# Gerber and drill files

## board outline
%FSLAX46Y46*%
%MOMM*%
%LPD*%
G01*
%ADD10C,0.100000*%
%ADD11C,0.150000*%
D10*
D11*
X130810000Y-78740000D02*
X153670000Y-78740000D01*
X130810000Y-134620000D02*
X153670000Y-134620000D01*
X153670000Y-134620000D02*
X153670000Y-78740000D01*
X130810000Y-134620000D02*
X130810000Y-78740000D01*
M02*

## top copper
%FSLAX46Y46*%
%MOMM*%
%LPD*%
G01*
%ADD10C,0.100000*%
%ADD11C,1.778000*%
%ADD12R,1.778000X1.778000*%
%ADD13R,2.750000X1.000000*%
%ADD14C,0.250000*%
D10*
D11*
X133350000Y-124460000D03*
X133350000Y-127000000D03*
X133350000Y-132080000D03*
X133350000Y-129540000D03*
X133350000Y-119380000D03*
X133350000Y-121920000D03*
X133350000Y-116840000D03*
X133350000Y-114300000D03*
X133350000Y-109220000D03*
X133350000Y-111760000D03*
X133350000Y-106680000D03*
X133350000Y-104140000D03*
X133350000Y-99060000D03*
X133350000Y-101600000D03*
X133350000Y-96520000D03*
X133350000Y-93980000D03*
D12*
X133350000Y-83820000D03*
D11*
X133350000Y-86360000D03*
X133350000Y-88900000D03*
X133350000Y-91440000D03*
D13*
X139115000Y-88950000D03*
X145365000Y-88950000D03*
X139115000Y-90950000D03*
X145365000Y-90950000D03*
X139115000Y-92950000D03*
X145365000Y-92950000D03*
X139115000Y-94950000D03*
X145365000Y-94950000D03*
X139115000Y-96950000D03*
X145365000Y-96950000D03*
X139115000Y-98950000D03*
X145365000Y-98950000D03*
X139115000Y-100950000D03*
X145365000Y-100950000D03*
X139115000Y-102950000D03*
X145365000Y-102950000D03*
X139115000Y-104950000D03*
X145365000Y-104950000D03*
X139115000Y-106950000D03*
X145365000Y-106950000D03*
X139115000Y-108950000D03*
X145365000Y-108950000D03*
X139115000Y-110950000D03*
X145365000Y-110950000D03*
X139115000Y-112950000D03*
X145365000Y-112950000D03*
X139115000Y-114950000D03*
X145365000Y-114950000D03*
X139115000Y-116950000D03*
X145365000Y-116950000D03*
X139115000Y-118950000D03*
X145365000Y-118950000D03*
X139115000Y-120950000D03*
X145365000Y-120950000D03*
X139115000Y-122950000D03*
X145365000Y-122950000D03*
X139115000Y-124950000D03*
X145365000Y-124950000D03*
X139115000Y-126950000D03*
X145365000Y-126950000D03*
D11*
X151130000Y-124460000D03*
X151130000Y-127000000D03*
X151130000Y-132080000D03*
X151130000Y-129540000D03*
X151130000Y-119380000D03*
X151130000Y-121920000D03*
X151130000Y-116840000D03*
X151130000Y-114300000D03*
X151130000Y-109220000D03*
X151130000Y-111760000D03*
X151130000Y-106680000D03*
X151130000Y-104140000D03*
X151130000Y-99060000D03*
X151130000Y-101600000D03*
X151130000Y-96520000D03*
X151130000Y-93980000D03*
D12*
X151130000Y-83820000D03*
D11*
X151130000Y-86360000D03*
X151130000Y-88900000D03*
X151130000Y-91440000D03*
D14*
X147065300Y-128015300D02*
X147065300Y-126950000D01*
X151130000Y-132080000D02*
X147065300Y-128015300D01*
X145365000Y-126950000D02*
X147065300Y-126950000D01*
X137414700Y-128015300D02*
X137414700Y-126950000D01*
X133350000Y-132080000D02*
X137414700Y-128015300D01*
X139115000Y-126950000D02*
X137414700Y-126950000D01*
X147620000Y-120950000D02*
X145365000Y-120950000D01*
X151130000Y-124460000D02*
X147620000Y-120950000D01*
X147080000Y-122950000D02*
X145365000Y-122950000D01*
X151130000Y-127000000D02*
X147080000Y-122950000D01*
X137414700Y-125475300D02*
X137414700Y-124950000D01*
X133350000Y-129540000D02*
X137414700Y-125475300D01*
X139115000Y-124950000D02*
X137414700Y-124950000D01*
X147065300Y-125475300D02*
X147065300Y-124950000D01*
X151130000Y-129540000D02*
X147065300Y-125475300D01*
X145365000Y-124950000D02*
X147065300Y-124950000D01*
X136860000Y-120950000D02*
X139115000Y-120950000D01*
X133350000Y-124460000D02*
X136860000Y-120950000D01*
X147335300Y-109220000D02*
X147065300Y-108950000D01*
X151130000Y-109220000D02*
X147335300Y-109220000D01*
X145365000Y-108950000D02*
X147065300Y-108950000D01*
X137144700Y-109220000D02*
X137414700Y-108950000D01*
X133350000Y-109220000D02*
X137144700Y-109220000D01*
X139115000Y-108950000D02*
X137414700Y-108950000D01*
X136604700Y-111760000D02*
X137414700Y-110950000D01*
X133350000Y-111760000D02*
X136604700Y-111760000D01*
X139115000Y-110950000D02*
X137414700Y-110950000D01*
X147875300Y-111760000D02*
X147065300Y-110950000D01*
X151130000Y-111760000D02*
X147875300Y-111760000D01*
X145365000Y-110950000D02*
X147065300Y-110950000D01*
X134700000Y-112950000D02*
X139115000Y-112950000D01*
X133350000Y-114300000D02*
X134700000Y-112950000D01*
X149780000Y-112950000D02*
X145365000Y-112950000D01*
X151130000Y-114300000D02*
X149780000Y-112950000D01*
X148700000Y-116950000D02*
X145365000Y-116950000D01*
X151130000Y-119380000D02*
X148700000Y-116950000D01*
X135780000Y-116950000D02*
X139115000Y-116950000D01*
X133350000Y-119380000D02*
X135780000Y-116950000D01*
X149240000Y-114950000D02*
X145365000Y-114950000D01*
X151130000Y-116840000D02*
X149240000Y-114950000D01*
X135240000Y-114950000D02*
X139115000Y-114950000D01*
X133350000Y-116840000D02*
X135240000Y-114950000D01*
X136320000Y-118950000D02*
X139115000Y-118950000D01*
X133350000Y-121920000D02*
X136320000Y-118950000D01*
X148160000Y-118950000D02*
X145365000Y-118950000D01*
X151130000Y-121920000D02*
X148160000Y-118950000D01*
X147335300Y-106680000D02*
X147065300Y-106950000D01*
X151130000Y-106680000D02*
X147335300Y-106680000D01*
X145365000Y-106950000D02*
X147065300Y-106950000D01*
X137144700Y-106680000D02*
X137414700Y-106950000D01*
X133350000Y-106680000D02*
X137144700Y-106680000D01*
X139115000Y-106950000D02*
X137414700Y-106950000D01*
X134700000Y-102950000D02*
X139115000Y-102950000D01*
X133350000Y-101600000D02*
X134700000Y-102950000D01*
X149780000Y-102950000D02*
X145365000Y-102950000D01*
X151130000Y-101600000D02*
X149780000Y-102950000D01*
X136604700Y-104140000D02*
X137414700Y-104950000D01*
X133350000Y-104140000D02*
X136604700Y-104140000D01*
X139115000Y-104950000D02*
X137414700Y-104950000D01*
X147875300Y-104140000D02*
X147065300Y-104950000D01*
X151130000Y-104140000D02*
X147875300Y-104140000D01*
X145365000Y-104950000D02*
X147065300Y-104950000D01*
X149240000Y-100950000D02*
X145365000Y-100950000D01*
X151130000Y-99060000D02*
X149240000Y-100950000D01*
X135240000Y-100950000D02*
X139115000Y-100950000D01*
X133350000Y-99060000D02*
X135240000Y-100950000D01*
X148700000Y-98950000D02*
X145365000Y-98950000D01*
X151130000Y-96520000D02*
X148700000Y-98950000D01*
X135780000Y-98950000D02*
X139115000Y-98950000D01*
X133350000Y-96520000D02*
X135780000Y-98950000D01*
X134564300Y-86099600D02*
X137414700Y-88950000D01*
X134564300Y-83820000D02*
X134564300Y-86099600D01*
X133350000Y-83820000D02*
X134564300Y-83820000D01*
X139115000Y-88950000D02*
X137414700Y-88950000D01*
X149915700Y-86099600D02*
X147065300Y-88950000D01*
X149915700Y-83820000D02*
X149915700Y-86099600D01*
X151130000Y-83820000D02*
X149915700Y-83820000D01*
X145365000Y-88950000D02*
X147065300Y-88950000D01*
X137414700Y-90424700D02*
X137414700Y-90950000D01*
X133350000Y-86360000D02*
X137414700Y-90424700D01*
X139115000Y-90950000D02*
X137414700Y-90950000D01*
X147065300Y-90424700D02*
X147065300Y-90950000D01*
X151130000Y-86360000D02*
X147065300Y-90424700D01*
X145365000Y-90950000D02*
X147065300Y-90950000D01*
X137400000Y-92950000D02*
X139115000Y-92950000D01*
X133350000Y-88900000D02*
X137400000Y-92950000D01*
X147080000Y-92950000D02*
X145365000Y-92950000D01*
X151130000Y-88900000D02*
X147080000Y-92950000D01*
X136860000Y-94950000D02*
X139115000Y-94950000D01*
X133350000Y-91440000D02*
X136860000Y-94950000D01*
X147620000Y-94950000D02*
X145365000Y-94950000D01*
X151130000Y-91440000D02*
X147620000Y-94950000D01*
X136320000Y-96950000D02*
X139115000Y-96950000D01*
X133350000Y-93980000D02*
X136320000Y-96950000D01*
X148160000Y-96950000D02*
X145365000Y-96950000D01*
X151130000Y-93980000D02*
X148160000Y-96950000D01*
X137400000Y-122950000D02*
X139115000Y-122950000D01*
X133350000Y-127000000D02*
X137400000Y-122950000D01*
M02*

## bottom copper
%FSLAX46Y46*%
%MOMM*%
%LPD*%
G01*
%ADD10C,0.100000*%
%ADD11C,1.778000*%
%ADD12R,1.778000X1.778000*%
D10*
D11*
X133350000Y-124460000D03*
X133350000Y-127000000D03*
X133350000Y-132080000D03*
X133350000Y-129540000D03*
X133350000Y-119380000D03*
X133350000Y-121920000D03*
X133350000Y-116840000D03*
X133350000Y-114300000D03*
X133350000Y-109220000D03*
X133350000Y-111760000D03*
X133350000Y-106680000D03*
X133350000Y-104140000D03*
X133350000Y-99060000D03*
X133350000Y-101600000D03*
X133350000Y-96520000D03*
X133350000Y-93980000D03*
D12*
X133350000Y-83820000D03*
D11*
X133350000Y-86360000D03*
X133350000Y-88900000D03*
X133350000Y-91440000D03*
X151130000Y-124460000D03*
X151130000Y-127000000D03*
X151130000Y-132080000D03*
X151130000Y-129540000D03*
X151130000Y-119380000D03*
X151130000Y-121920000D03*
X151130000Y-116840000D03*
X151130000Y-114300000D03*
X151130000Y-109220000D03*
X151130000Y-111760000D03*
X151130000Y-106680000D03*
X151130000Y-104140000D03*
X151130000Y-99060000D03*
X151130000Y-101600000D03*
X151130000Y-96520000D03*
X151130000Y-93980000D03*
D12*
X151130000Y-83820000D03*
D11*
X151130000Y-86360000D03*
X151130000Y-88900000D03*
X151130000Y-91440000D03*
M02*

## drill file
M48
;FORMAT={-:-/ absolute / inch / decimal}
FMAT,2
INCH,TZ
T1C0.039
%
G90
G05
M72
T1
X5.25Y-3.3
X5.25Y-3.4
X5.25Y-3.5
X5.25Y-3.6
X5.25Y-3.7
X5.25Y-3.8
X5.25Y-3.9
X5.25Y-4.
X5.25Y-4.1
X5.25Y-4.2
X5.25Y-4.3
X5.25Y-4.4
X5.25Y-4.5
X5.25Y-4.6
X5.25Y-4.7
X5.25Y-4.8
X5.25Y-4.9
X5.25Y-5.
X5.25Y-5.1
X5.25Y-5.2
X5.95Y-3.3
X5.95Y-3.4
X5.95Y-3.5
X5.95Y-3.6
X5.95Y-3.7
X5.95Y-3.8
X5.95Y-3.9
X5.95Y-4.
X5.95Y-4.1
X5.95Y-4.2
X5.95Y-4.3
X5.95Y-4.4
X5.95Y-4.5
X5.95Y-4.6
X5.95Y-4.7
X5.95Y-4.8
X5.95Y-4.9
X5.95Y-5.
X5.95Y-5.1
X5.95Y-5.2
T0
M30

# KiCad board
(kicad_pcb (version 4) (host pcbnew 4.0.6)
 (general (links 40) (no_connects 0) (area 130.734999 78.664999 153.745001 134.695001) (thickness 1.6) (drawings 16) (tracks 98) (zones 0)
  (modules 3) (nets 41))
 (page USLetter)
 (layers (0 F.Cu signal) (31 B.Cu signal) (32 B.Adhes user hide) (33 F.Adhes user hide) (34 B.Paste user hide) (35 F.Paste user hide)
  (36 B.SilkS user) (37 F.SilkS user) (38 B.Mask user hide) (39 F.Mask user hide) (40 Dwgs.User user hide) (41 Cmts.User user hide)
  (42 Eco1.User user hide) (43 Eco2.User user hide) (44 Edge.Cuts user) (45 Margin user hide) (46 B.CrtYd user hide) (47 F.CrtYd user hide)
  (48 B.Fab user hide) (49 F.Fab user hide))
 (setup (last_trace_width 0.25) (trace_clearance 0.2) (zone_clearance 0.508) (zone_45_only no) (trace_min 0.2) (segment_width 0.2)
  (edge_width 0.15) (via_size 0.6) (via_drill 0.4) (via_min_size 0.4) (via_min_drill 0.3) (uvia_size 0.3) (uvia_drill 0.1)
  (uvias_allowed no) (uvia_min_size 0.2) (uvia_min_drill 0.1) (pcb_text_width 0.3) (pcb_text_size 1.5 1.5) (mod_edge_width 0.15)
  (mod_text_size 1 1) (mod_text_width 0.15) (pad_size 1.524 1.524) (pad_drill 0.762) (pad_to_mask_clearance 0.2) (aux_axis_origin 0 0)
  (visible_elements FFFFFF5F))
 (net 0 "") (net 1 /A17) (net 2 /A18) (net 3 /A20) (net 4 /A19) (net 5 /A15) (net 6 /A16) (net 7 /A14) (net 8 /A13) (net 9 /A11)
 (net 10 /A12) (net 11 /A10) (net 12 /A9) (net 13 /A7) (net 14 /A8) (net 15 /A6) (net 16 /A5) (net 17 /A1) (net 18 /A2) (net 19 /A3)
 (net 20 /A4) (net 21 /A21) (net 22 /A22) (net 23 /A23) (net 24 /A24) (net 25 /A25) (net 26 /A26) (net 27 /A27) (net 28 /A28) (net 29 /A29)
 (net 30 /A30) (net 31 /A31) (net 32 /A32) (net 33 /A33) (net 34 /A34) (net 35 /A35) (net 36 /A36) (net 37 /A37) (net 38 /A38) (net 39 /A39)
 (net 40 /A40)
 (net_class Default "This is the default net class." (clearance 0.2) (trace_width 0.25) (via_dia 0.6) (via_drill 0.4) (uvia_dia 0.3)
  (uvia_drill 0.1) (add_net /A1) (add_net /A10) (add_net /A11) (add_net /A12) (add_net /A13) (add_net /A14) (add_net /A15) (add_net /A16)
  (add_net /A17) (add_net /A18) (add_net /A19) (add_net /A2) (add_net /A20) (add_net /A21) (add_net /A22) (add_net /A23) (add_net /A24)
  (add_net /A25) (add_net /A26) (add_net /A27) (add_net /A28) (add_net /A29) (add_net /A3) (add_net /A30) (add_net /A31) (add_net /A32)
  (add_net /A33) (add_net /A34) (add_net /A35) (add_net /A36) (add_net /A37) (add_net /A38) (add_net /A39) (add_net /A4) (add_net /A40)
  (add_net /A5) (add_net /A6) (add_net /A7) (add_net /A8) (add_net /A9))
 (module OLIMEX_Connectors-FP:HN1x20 (layer F.Cu) (at 133.35 107.95 270) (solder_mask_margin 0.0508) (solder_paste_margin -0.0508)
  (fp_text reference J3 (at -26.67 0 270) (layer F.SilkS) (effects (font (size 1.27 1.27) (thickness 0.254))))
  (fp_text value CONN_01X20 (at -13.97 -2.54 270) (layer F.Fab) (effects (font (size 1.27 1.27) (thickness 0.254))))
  (pad 17 thru_hole circle (at 16.51 0 270) (size 1.778 1.778) (drill 1) (layers *.Cu *.Mask) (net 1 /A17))
  (pad 18 thru_hole circle (at 19.05 0 270) (size 1.778 1.778) (drill 1) (layers *.Cu *.Mask) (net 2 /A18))
  (pad 20 thru_hole circle (at 24.13 0 270) (size 1.778 1.778) (drill 1) (layers *.Cu *.Mask) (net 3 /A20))
  (pad 19 thru_hole circle (at 21.59 0 270) (size 1.778 1.778) (drill 1) (layers *.Cu *.Mask) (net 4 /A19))
  (pad 15 thru_hole circle (at 11.43 0 270) (size 1.778 1.778) (drill 1) (layers *.Cu *.Mask) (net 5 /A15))
  (pad 16 thru_hole circle (at 13.97 0 270) (size 1.778 1.778) (drill 1) (layers *.Cu *.Mask) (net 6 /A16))
  (pad 14 thru_hole circle (at 8.89 0 270) (size 1.778 1.778) (drill 1) (layers *.Cu *.Mask) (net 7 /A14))
  (pad 13 thru_hole circle (at 6.35 0 270) (size 1.778 1.778) (drill 1) (layers *.Cu *.Mask) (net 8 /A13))
  (pad 11 thru_hole circle (at 1.27 0 270) (size 1.778 1.778) (drill 1) (layers *.Cu *.Mask) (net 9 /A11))
  (pad 12 thru_hole circle (at 3.81 0 270) (size 1.778 1.778) (drill 1) (layers *.Cu *.Mask) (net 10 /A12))
  (pad 10 thru_hole circle (at -1.27 0 270) (size 1.778 1.778) (drill 1) (layers *.Cu *.Mask) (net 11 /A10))
  (pad 9 thru_hole circle (at -3.81 0 270) (size 1.778 1.778) (drill 1) (layers *.Cu *.Mask) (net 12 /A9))
  (pad 7 thru_hole circle (at -8.89 0 270) (size 1.778 1.778) (drill 1) (layers *.Cu *.Mask) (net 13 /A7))
  (pad 8 thru_hole circle (at -6.35 0 270) (size 1.778 1.778) (drill 1) (layers *.Cu *.Mask) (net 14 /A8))
  (pad 6 thru_hole circle (at -11.43 0 270) (size 1.778 1.778) (drill 1) (layers *.Cu *.Mask) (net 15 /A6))
  (pad 5 thru_hole circle (at -13.97 0 270) (size 1.778 1.778) (drill 1) (layers *.Cu *.Mask) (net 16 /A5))
  (pad 1 thru_hole rect (at -24.13 0 270) (size 1.778 1.778) (drill 1) (layers *.Cu *.Mask) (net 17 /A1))
  (pad 2 thru_hole circle (at -21.59 0 270) (size 1.778 1.778) (drill 1) (layers *.Cu *.Mask) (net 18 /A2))
  (pad 3 thru_hole circle (at -19.05 0 270) (size 1.778 1.778) (drill 1) (layers *.Cu *.Mask) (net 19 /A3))
  (pad 4 thru_hole circle (at -16.51 0 270) (size 1.778 1.778) (drill 1) (layers *.Cu *.Mask) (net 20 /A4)))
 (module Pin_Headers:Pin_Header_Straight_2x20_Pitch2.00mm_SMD (layer F.Cu) (at 142.24 107.95)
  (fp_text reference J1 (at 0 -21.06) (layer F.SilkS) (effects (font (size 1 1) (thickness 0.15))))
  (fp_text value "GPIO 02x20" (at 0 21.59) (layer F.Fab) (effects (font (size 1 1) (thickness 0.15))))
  (pad 1 smd rect (at -3.125 -19) (size 2.75 1) (layers F.Cu F.Mask) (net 17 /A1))
  (pad 2 smd rect (at 3.125 -19) (size 2.75 1) (layers F.Cu F.Mask) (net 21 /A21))
  (pad 3 smd rect (at -3.125 -17) (size 2.75 1) (layers F.Cu F.Mask) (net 18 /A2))
  (pad 4 smd rect (at 3.125 -17) (size 2.75 1) (layers F.Cu F.Mask) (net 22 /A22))
  (pad 5 smd rect (at -3.125 -15) (size 2.75 1) (layers F.Cu F.Mask) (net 19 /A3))
  (pad 6 smd rect (at 3.125 -15) (size 2.75 1) (layers F.Cu F.Mask) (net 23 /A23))
  (pad 7 smd rect (at -3.125 -13) (size 2.75 1) (layers F.Cu F.Mask) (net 20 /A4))
  (pad 8 smd rect (at 3.125 -13) (size 2.75 1) (layers F.Cu F.Mask) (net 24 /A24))
  (pad 9 smd rect (at -3.125 -11) (size 2.75 1) (layers F.Cu F.Mask) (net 16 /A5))
  (pad 10 smd rect (at 3.125 -11) (size 2.75 1) (layers F.Cu F.Mask) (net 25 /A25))
  (pad 11 smd rect (at -3.125 -9) (size 2.75 1) (layers F.Cu F.Mask) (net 15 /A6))
  (pad 12 smd rect (at 3.125 -9) (size 2.75 1) (layers F.Cu F.Mask) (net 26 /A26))
  (pad 13 smd rect (at -3.125 -7) (size 2.75 1) (layers F.Cu F.Mask) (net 13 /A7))
  (pad 14 smd rect (at 3.125 -7) (size 2.75 1) (layers F.Cu F.Mask) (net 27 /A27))
  (pad 15 smd rect (at -3.125 -5) (size 2.75 1) (layers F.Cu F.Mask) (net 14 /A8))
  (pad 16 smd rect (at 3.125 -5) (size 2.75 1) (layers F.Cu F.Mask) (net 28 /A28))
  (pad 17 smd rect (at -3.125 -3) (size 2.75 1) (layers F.Cu F.Mask) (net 12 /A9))
  (pad 18 smd rect (at 3.125 -3) (size 2.75 1) (layers F.Cu F.Mask) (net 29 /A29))
  (pad 19 smd rect (at -3.125 -1) (size 2.75 1) (layers F.Cu F.Mask) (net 11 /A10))
  (pad 20 smd rect (at 3.125 -1) (size 2.75 1) (layers F.Cu F.Mask) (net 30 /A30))
  (pad 21 smd rect (at -3.125 1) (size 2.75 1) (layers F.Cu F.Mask) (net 9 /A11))
  (pad 22 smd rect (at 3.125 1) (size 2.75 1) (layers F.Cu F.Mask) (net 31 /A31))
  (pad 23 smd rect (at -3.125 3) (size 2.75 1) (layers F.Cu F.Mask) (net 10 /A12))
  (pad 24 smd rect (at 3.125 3) (size 2.75 1) (layers F.Cu F.Mask) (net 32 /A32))
  (pad 25 smd rect (at -3.125 5) (size 2.75 1) (layers F.Cu F.Mask) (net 8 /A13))
  (pad 26 smd rect (at 3.125 5) (size 2.75 1) (layers F.Cu F.Mask) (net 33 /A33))
  (pad 27 smd rect (at -3.125 7) (size 2.75 1) (layers F.Cu F.Mask) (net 7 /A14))
  (pad 28 smd rect (at 3.125 7) (size 2.75 1) (layers F.Cu F.Mask) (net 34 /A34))
  (pad 29 smd rect (at -3.125 9) (size 2.75 1) (layers F.Cu F.Mask) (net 5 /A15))
  (pad 30 smd rect (at 3.125 9) (size 2.75 1) (layers F.Cu F.Mask) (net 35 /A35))
  (pad 31 smd rect (at -3.125 11) (size 2.75 1) (layers F.Cu F.Mask) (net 6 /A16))
  (pad 32 smd rect (at 3.125 11) (size 2.75 1) (layers F.Cu F.Mask) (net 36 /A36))
  (pad 33 smd rect (at -3.125 13) (size 2.75 1) (layers F.Cu F.Mask) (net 1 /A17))
  (pad 34 smd rect (at 3.125 13) (size 2.75 1) (layers F.Cu F.Mask) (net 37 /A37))
  (pad 35 smd rect (at -3.125 15) (size 2.75 1) (layers F.Cu F.Mask) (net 2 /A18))
  (pad 36 smd rect (at 3.125 15) (size 2.75 1) (layers F.Cu F.Mask) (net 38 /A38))
  (pad 37 smd rect (at -3.125 17) (size 2.75 1) (layers F.Cu F.Mask) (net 4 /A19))
  (pad 38 smd rect (at 3.125 17) (size 2.75 1) (layers F.Cu F.Mask) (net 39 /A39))
  (pad 39 smd rect (at -3.125 19) (size 2.75 1) (layers F.Cu F.Mask) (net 3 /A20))
  (pad 40 smd rect (at 3.125 19) (size 2.75 1) (layers F.Cu F.Mask) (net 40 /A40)))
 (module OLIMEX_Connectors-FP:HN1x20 (layer F.Cu) (at 151.13 107.95 270) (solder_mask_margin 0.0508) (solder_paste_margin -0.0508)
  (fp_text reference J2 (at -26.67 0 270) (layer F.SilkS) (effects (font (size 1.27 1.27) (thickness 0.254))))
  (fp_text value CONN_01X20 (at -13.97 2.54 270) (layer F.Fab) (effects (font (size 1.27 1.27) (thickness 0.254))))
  (pad 17 thru_hole circle (at 16.51 0 270) (size 1.778 1.778) (drill 1) (layers *.Cu *.Mask) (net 37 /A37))
  (pad 18 thru_hole circle (at 19.05 0 270) (size 1.778 1.778) (drill 1) (layers *.Cu *.Mask) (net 38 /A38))
  (pad 20 thru_hole circle (at 24.13 0 270) (size 1.778 1.778) (drill 1) (layers *.Cu *.Mask) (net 40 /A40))
  (pad 19 thru_hole circle (at 21.59 0 270) (size 1.778 1.778) (drill 1) (layers *.Cu *.Mask) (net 39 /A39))
  (pad 15 thru_hole circle (at 11.43 0 270) (size 1.778 1.778) (drill 1) (layers *.Cu *.Mask) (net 35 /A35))
  (pad 16 thru_hole circle (at 13.97 0 270) (size 1.778 1.778) (drill 1) (layers *.Cu *.Mask) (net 36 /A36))
  (pad 14 thru_hole circle (at 8.89 0 270) (size 1.778 1.778) (drill 1) (layers *.Cu *.Mask) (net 34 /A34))
  (pad 13 thru_hole circle (at 6.35 0 270) (size 1.778 1.778) (drill 1) (layers *.Cu *.Mask) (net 33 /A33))
  (pad 11 thru_hole circle (at 1.27 0 270) (size 1.778 1.778) (drill 1) (layers *.Cu *.Mask) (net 31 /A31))
  (pad 12 thru_hole circle (at 3.81 0 270) (size 1.778 1.778) (drill 1) (layers *.Cu *.Mask) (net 32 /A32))
  (pad 10 thru_hole circle (at -1.27 0 270) (size 1.778 1.778) (drill 1) (layers *.Cu *.Mask) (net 30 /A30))
  (pad 9 thru_hole circle (at -3.81 0 270) (size 1.778 1.778) (drill 1) (layers *.Cu *.Mask) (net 29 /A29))
  (pad 7 thru_hole circle (at -8.89 0 270) (size 1.778 1.778) (drill 1) (layers *.Cu *.Mask) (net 27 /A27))
  (pad 8 thru_hole circle (at -6.35 0 270) (size 1.778 1.778) (drill 1) (layers *.Cu *.Mask) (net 28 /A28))
  (pad 6 thru_hole circle (at -11.43 0 270) (size 1.778 1.778) (drill 1) (layers *.Cu *.Mask) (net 26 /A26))
  (pad 5 thru_hole circle (at -13.97 0 270) (size 1.778 1.778) (drill 1) (layers *.Cu *.Mask) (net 25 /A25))
  (pad 1 thru_hole rect (at -24.13 0 270) (size 1.778 1.778) (drill 1) (layers *.Cu *.Mask) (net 21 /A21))
  (pad 2 thru_hole circle (at -21.59 0 270) (size 1.778 1.778) (drill 1) (layers *.Cu *.Mask) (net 22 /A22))
  (pad 3 thru_hole circle (at -19.05 0 270) (size 1.778 1.778) (drill 1) (layers *.Cu *.Mask) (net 23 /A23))
  (pad 4 thru_hole circle (at -16.51 0 270) (size 1.778 1.778) (drill 1) (layers *.Cu *.Mask) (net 24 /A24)))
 (gr_line (start 130.81 78.74) (end 153.67 78.74) (angle 90) (layer Edge.Cuts) (width 0.15))
 (gr_line (start 130.81 134.62) (end 153.67 134.62) (angle 90) (layer Edge.Cuts) (width 0.15))
 (gr_line (start 153.67 134.62) (end 153.67 78.74) (angle 90) (layer Edge.Cuts) (width 0.15))
 (gr_line (start 130.81 134.62) (end 130.81 78.74) (angle 90) (layer Edge.Cuts) (width 0.15))
 (segment (start 147.0653 128.0153) (end 147.0653 126.95) (width 0.25) (layer F.Cu) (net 40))
 (segment (start 151.13 132.08) (end 147.0653 128.0153) (width 0.25) (layer F.Cu) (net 40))
 (segment (start 145.365 126.95) (end 147.0653 126.95) (width 0.25) (layer F.Cu) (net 40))
 (segment (start 137.4147 128.0153) (end 137.4147 126.95) (width 0.25) (layer F.Cu) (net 3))
 (segment (start 133.35 132.08) (end 137.4147 128.0153) (width 0.25) (layer F.Cu) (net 3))
 (segment (start 139.115 126.95) (end 137.4147 126.95) (width 0.25) (layer F.Cu) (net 3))
 (segment (start 147.62 120.95) (end 145.365 120.95) (width 0.25) (layer F.Cu) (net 37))
 (segment (start 151.13 124.46) (end 147.62 120.95) (width 0.25) (layer F.Cu) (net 37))
 (segment (start 147.08 122.95) (end 145.365 122.95) (width 0.25) (layer F.Cu) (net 38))
 (segment (start 151.13 127) (end 147.08 122.95) (width 0.25) (layer F.Cu) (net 38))
 (segment (start 137.4147 125.4753) (end 137.4147 124.95) (width 0.25) (layer F.Cu) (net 4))
 (segment (start 133.35 129.54) (end 137.4147 125.4753) (width 0.25) (layer F.Cu) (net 4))
 (segment (start 139.115 124.95) (end 137.4147 124.95) (width 0.25) (layer F.Cu) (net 4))
 (segment (start 147.0653 125.4753) (end 147.0653 124.95) (width 0.25) (layer F.Cu) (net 39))
 (segment (start 151.13 129.54) (end 147.0653 125.4753) (width 0.25) (layer F.Cu) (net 39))
 (segment (start 145.365 124.95) (end 147.0653 124.95) (width 0.25) (layer F.Cu) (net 39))
 (segment (start 136.86 120.95) (end 139.115 120.95) (width 0.25) (layer F.Cu) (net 1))
 (segment (start 133.35 124.46) (end 136.86 120.95) (width 0.25) (layer F.Cu) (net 1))
 (segment (start 147.3353 109.22) (end 147.0653 108.95) (width 0.25) (layer F.Cu) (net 31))
 (segment (start 151.13 109.22) (end 147.3353 109.22) (width 0.25) (layer F.Cu) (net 31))
 (segment (start 145.365 108.95) (end 147.0653 108.95) (width 0.25) (layer F.Cu) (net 31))
 (segment (start 137.1447 109.22) (end 137.4147 108.95) (width 0.25) (layer F.Cu) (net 9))
 (segment (start 133.35 109.22) (end 137.1447 109.22) (width 0.25) (layer F.Cu) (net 9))
 (segment (start 139.115 108.95) (end 137.4147 108.95) (width 0.25) (layer F.Cu) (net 9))
 (segment (start 136.6047 111.76) (end 137.4147 110.95) (width 0.25) (layer F.Cu) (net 10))
 (segment (start 133.35 111.76) (end 136.6047 111.76) (width 0.25) (layer F.Cu) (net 10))
 (segment (start 139.115 110.95) (end 137.4147 110.95) (width 0.25) (layer F.Cu) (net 10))
 (segment (start 147.8753 111.76) (end 147.0653 110.95) (width 0.25) (layer F.Cu) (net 32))
 (segment (start 151.13 111.76) (end 147.8753 111.76) (width 0.25) (layer F.Cu) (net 32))
 (segment (start 145.365 110.95) (end 147.0653 110.95) (width 0.25) (layer F.Cu) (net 32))
 (segment (start 134.7 112.95) (end 139.115 112.95) (width 0.25) (layer F.Cu) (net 8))
 (segment (start 133.35 114.3) (end 134.7 112.95) (width 0.25) (layer F.Cu) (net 8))
 (segment (start 149.78 112.95) (end 145.365 112.95) (width 0.25) (layer F.Cu) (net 33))
 (segment (start 151.13 114.3) (end 149.78 112.95) (width 0.25) (layer F.Cu) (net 33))
 (segment (start 148.7 116.95) (end 145.365 116.95) (width 0.25) (layer F.Cu) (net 35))
 (segment (start 151.13 119.38) (end 148.7 116.95) (width 0.25) (layer F.Cu) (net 35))
 (segment (start 135.78 116.95) (end 139.115 116.95) (width 0.25) (layer F.Cu) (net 5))
 (segment (start 133.35 119.38) (end 135.78 116.95) (width 0.25) (layer F.Cu) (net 5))
 (segment (start 149.24 114.95) (end 145.365 114.95) (width 0.25) (layer F.Cu) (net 34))
 (segment (start 151.13 116.84) (end 149.24 114.95) (width 0.25) (layer F.Cu) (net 34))
 (segment (start 135.24 114.95) (end 139.115 114.95) (width 0.25) (layer F.Cu) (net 7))
 (segment (start 133.35 116.84) (end 135.24 114.95) (width 0.25) (layer F.Cu) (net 7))
 (segment (start 136.32 118.95) (end 139.115 118.95) (width 0.25) (layer F.Cu) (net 6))
 (segment (start 133.35 121.92) (end 136.32 118.95) (width 0.25) (layer F.Cu) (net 6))
 (segment (start 148.16 118.95) (end 145.365 118.95) (width 0.25) (layer F.Cu) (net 36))
 (segment (start 151.13 121.92) (end 148.16 118.95) (width 0.25) (layer F.Cu) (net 36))
 (segment (start 147.3353 106.68) (end 147.0653 106.95) (width 0.25) (layer F.Cu) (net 30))
 (segment (start 151.13 106.68) (end 147.3353 106.68) (width 0.25) (layer F.Cu) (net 30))
 (segment (start 145.365 106.95) (end 147.0653 106.95) (width 0.25) (layer F.Cu) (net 30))
 (segment (start 137.1447 106.68) (end 137.4147 106.95) (width 0.25) (layer F.Cu) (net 11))
 (segment (start 133.35 106.68) (end 137.1447 106.68) (width 0.25) (layer F.Cu) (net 11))
 (segment (start 139.115 106.95) (end 137.4147 106.95) (width 0.25) (layer F.Cu) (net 11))
 (segment (start 134.7 102.95) (end 139.115 102.95) (width 0.25) (layer F.Cu) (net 14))
 (segment (start 133.35 101.6) (end 134.7 102.95) (width 0.25) (layer F.Cu) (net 14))
 (segment (start 149.78 102.95) (end 145.365 102.95) (width 0.25) (layer F.Cu) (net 28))
 (segment (start 151.13 101.6) (end 149.78 102.95) (width 0.25) (layer F.Cu) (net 28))
 (segment (start 136.6047 104.14) (end 137.4147 104.95) (width 0.25) (layer F.Cu) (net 12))
 (segment (start 133.35 104.14) (end 136.6047 104.14) (width 0.25) (layer F.Cu) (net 12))
 (segment (start 139.115 104.95) (end 137.4147 104.95) (width 0.25) (layer F.Cu) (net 12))
 (segment (start 147.8753 104.14) (end 147.0653 104.95) (width 0.25) (layer F.Cu) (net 29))
 (segment (start 151.13 104.14) (end 147.8753 104.14) (width 0.25) (layer F.Cu) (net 29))
 (segment (start 145.365 104.95) (end 147.0653 104.95) (width 0.25) (layer F.Cu) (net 29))
 (segment (start 149.24 100.95) (end 145.365 100.95) (width 0.25) (layer F.Cu) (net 27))
 (segment (start 151.13 99.06) (end 149.24 100.95) (width 0.25) (layer F.Cu) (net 27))
 (segment (start 135.24 100.95) (end 139.115 100.95) (width 0.25) (layer F.Cu) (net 13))
 (segment (start 133.35 99.06) (end 135.24 100.95) (width 0.25) (layer F.Cu) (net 13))
 (segment (start 148.7 98.95) (end 145.365 98.95) (width 0.25) (layer F.Cu) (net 26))
 (segment (start 151.13 96.52) (end 148.7 98.95) (width 0.25) (layer F.Cu) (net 26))
 (segment (start 135.78 98.95) (end 139.115 98.95) (width 0.25) (layer F.Cu) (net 15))
 (segment (start 133.35 96.52) (end 135.78 98.95) (width 0.25) (layer F.Cu) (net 15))
 (segment (start 134.5643 86.0996) (end 137.4147 88.95) (width 0.25) (layer F.Cu) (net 17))
 (segment (start 134.5643 83.82) (end 134.5643 86.0996) (width 0.25) (layer F.Cu) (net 17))
 (segment (start 133.35 83.82) (end 134.5643 83.82) (width 0.25) (layer F.Cu) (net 17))
 (segment (start 139.115 88.95) (end 137.4147 88.95) (width 0.25) (layer F.Cu) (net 17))
 (segment (start 149.9157 86.0996) (end 147.0653 88.95) (width 0.25) (layer F.Cu) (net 21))
 (segment (start 149.9157 83.82) (end 149.9157 86.0996) (width 0.25) (layer F.Cu) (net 21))
 (segment (start 151.13 83.82) (end 149.9157 83.82) (width 0.25) (layer F.Cu) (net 21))
 (segment (start 145.365 88.95) (end 147.0653 88.95) (width 0.25) (layer F.Cu) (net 21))
 (segment (start 137.4147 90.4247) (end 137.4147 90.95) (width 0.25) (layer F.Cu) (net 18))
 (segment (start 133.35 86.36) (end 137.4147 90.4247) (width 0.25) (layer F.Cu) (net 18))
 (segment (start 139.115 90.95) (end 137.4147 90.95) (width 0.25) (layer F.Cu) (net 18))
 (segment (start 147.0653 90.4247) (end 147.0653 90.95) (width 0.25) (layer F.Cu) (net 22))
 (segment (start 151.13 86.36) (end 147.0653 90.4247) (width 0.25) (layer F.Cu) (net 22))
 (segment (start 145.365 90.95) (end 147.0653 90.95) (width 0.25) (layer F.Cu) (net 22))
 (segment (start 137.4 92.95) (end 139.115 92.95) (width 0.25) (layer F.Cu) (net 19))
 (segment (start 133.35 88.9) (end 137.4 92.95) (width 0.25) (layer F.Cu) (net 19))
 (segment (start 147.08 92.95) (end 145.365 92.95) (width 0.25) (layer F.Cu) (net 23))
 (segment (start 151.13 88.9) (end 147.08 92.95) (width 0.25) (layer F.Cu) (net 23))
 (segment (start 136.86 94.95) (end 139.115 94.95) (width 0.25) (layer F.Cu) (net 20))
 (segment (start 133.35 91.44) (end 136.86 94.95) (width 0.25) (layer F.Cu) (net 20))
 (segment (start 147.62 94.95) (end 145.365 94.95) (width 0.25) (layer F.Cu) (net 24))
 (segment (start 151.13 91.44) (end 147.62 94.95) (width 0.25) (layer F.Cu) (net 24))
 (segment (start 136.32 96.95) (end 139.115 96.95) (width 0.25) (layer F.Cu) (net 16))
 (segment (start 133.35 93.98) (end 136.32 96.95) (width 0.25) (layer F.Cu) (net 16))
 (segment (start 148.16 96.95) (end 145.365 96.95) (width 0.25) (layer F.Cu) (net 25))
 (segment (start 151.13 93.98) (end 148.16 96.95) (width 0.25) (layer F.Cu) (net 25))
 (segment (start 137.4 122.95) (end 139.115 122.95) (width 0.25) (layer F.Cu) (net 2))
 (segment (start 133.35 127) (end 137.4 122.95) (width 0.25) (layer F.Cu) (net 2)))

